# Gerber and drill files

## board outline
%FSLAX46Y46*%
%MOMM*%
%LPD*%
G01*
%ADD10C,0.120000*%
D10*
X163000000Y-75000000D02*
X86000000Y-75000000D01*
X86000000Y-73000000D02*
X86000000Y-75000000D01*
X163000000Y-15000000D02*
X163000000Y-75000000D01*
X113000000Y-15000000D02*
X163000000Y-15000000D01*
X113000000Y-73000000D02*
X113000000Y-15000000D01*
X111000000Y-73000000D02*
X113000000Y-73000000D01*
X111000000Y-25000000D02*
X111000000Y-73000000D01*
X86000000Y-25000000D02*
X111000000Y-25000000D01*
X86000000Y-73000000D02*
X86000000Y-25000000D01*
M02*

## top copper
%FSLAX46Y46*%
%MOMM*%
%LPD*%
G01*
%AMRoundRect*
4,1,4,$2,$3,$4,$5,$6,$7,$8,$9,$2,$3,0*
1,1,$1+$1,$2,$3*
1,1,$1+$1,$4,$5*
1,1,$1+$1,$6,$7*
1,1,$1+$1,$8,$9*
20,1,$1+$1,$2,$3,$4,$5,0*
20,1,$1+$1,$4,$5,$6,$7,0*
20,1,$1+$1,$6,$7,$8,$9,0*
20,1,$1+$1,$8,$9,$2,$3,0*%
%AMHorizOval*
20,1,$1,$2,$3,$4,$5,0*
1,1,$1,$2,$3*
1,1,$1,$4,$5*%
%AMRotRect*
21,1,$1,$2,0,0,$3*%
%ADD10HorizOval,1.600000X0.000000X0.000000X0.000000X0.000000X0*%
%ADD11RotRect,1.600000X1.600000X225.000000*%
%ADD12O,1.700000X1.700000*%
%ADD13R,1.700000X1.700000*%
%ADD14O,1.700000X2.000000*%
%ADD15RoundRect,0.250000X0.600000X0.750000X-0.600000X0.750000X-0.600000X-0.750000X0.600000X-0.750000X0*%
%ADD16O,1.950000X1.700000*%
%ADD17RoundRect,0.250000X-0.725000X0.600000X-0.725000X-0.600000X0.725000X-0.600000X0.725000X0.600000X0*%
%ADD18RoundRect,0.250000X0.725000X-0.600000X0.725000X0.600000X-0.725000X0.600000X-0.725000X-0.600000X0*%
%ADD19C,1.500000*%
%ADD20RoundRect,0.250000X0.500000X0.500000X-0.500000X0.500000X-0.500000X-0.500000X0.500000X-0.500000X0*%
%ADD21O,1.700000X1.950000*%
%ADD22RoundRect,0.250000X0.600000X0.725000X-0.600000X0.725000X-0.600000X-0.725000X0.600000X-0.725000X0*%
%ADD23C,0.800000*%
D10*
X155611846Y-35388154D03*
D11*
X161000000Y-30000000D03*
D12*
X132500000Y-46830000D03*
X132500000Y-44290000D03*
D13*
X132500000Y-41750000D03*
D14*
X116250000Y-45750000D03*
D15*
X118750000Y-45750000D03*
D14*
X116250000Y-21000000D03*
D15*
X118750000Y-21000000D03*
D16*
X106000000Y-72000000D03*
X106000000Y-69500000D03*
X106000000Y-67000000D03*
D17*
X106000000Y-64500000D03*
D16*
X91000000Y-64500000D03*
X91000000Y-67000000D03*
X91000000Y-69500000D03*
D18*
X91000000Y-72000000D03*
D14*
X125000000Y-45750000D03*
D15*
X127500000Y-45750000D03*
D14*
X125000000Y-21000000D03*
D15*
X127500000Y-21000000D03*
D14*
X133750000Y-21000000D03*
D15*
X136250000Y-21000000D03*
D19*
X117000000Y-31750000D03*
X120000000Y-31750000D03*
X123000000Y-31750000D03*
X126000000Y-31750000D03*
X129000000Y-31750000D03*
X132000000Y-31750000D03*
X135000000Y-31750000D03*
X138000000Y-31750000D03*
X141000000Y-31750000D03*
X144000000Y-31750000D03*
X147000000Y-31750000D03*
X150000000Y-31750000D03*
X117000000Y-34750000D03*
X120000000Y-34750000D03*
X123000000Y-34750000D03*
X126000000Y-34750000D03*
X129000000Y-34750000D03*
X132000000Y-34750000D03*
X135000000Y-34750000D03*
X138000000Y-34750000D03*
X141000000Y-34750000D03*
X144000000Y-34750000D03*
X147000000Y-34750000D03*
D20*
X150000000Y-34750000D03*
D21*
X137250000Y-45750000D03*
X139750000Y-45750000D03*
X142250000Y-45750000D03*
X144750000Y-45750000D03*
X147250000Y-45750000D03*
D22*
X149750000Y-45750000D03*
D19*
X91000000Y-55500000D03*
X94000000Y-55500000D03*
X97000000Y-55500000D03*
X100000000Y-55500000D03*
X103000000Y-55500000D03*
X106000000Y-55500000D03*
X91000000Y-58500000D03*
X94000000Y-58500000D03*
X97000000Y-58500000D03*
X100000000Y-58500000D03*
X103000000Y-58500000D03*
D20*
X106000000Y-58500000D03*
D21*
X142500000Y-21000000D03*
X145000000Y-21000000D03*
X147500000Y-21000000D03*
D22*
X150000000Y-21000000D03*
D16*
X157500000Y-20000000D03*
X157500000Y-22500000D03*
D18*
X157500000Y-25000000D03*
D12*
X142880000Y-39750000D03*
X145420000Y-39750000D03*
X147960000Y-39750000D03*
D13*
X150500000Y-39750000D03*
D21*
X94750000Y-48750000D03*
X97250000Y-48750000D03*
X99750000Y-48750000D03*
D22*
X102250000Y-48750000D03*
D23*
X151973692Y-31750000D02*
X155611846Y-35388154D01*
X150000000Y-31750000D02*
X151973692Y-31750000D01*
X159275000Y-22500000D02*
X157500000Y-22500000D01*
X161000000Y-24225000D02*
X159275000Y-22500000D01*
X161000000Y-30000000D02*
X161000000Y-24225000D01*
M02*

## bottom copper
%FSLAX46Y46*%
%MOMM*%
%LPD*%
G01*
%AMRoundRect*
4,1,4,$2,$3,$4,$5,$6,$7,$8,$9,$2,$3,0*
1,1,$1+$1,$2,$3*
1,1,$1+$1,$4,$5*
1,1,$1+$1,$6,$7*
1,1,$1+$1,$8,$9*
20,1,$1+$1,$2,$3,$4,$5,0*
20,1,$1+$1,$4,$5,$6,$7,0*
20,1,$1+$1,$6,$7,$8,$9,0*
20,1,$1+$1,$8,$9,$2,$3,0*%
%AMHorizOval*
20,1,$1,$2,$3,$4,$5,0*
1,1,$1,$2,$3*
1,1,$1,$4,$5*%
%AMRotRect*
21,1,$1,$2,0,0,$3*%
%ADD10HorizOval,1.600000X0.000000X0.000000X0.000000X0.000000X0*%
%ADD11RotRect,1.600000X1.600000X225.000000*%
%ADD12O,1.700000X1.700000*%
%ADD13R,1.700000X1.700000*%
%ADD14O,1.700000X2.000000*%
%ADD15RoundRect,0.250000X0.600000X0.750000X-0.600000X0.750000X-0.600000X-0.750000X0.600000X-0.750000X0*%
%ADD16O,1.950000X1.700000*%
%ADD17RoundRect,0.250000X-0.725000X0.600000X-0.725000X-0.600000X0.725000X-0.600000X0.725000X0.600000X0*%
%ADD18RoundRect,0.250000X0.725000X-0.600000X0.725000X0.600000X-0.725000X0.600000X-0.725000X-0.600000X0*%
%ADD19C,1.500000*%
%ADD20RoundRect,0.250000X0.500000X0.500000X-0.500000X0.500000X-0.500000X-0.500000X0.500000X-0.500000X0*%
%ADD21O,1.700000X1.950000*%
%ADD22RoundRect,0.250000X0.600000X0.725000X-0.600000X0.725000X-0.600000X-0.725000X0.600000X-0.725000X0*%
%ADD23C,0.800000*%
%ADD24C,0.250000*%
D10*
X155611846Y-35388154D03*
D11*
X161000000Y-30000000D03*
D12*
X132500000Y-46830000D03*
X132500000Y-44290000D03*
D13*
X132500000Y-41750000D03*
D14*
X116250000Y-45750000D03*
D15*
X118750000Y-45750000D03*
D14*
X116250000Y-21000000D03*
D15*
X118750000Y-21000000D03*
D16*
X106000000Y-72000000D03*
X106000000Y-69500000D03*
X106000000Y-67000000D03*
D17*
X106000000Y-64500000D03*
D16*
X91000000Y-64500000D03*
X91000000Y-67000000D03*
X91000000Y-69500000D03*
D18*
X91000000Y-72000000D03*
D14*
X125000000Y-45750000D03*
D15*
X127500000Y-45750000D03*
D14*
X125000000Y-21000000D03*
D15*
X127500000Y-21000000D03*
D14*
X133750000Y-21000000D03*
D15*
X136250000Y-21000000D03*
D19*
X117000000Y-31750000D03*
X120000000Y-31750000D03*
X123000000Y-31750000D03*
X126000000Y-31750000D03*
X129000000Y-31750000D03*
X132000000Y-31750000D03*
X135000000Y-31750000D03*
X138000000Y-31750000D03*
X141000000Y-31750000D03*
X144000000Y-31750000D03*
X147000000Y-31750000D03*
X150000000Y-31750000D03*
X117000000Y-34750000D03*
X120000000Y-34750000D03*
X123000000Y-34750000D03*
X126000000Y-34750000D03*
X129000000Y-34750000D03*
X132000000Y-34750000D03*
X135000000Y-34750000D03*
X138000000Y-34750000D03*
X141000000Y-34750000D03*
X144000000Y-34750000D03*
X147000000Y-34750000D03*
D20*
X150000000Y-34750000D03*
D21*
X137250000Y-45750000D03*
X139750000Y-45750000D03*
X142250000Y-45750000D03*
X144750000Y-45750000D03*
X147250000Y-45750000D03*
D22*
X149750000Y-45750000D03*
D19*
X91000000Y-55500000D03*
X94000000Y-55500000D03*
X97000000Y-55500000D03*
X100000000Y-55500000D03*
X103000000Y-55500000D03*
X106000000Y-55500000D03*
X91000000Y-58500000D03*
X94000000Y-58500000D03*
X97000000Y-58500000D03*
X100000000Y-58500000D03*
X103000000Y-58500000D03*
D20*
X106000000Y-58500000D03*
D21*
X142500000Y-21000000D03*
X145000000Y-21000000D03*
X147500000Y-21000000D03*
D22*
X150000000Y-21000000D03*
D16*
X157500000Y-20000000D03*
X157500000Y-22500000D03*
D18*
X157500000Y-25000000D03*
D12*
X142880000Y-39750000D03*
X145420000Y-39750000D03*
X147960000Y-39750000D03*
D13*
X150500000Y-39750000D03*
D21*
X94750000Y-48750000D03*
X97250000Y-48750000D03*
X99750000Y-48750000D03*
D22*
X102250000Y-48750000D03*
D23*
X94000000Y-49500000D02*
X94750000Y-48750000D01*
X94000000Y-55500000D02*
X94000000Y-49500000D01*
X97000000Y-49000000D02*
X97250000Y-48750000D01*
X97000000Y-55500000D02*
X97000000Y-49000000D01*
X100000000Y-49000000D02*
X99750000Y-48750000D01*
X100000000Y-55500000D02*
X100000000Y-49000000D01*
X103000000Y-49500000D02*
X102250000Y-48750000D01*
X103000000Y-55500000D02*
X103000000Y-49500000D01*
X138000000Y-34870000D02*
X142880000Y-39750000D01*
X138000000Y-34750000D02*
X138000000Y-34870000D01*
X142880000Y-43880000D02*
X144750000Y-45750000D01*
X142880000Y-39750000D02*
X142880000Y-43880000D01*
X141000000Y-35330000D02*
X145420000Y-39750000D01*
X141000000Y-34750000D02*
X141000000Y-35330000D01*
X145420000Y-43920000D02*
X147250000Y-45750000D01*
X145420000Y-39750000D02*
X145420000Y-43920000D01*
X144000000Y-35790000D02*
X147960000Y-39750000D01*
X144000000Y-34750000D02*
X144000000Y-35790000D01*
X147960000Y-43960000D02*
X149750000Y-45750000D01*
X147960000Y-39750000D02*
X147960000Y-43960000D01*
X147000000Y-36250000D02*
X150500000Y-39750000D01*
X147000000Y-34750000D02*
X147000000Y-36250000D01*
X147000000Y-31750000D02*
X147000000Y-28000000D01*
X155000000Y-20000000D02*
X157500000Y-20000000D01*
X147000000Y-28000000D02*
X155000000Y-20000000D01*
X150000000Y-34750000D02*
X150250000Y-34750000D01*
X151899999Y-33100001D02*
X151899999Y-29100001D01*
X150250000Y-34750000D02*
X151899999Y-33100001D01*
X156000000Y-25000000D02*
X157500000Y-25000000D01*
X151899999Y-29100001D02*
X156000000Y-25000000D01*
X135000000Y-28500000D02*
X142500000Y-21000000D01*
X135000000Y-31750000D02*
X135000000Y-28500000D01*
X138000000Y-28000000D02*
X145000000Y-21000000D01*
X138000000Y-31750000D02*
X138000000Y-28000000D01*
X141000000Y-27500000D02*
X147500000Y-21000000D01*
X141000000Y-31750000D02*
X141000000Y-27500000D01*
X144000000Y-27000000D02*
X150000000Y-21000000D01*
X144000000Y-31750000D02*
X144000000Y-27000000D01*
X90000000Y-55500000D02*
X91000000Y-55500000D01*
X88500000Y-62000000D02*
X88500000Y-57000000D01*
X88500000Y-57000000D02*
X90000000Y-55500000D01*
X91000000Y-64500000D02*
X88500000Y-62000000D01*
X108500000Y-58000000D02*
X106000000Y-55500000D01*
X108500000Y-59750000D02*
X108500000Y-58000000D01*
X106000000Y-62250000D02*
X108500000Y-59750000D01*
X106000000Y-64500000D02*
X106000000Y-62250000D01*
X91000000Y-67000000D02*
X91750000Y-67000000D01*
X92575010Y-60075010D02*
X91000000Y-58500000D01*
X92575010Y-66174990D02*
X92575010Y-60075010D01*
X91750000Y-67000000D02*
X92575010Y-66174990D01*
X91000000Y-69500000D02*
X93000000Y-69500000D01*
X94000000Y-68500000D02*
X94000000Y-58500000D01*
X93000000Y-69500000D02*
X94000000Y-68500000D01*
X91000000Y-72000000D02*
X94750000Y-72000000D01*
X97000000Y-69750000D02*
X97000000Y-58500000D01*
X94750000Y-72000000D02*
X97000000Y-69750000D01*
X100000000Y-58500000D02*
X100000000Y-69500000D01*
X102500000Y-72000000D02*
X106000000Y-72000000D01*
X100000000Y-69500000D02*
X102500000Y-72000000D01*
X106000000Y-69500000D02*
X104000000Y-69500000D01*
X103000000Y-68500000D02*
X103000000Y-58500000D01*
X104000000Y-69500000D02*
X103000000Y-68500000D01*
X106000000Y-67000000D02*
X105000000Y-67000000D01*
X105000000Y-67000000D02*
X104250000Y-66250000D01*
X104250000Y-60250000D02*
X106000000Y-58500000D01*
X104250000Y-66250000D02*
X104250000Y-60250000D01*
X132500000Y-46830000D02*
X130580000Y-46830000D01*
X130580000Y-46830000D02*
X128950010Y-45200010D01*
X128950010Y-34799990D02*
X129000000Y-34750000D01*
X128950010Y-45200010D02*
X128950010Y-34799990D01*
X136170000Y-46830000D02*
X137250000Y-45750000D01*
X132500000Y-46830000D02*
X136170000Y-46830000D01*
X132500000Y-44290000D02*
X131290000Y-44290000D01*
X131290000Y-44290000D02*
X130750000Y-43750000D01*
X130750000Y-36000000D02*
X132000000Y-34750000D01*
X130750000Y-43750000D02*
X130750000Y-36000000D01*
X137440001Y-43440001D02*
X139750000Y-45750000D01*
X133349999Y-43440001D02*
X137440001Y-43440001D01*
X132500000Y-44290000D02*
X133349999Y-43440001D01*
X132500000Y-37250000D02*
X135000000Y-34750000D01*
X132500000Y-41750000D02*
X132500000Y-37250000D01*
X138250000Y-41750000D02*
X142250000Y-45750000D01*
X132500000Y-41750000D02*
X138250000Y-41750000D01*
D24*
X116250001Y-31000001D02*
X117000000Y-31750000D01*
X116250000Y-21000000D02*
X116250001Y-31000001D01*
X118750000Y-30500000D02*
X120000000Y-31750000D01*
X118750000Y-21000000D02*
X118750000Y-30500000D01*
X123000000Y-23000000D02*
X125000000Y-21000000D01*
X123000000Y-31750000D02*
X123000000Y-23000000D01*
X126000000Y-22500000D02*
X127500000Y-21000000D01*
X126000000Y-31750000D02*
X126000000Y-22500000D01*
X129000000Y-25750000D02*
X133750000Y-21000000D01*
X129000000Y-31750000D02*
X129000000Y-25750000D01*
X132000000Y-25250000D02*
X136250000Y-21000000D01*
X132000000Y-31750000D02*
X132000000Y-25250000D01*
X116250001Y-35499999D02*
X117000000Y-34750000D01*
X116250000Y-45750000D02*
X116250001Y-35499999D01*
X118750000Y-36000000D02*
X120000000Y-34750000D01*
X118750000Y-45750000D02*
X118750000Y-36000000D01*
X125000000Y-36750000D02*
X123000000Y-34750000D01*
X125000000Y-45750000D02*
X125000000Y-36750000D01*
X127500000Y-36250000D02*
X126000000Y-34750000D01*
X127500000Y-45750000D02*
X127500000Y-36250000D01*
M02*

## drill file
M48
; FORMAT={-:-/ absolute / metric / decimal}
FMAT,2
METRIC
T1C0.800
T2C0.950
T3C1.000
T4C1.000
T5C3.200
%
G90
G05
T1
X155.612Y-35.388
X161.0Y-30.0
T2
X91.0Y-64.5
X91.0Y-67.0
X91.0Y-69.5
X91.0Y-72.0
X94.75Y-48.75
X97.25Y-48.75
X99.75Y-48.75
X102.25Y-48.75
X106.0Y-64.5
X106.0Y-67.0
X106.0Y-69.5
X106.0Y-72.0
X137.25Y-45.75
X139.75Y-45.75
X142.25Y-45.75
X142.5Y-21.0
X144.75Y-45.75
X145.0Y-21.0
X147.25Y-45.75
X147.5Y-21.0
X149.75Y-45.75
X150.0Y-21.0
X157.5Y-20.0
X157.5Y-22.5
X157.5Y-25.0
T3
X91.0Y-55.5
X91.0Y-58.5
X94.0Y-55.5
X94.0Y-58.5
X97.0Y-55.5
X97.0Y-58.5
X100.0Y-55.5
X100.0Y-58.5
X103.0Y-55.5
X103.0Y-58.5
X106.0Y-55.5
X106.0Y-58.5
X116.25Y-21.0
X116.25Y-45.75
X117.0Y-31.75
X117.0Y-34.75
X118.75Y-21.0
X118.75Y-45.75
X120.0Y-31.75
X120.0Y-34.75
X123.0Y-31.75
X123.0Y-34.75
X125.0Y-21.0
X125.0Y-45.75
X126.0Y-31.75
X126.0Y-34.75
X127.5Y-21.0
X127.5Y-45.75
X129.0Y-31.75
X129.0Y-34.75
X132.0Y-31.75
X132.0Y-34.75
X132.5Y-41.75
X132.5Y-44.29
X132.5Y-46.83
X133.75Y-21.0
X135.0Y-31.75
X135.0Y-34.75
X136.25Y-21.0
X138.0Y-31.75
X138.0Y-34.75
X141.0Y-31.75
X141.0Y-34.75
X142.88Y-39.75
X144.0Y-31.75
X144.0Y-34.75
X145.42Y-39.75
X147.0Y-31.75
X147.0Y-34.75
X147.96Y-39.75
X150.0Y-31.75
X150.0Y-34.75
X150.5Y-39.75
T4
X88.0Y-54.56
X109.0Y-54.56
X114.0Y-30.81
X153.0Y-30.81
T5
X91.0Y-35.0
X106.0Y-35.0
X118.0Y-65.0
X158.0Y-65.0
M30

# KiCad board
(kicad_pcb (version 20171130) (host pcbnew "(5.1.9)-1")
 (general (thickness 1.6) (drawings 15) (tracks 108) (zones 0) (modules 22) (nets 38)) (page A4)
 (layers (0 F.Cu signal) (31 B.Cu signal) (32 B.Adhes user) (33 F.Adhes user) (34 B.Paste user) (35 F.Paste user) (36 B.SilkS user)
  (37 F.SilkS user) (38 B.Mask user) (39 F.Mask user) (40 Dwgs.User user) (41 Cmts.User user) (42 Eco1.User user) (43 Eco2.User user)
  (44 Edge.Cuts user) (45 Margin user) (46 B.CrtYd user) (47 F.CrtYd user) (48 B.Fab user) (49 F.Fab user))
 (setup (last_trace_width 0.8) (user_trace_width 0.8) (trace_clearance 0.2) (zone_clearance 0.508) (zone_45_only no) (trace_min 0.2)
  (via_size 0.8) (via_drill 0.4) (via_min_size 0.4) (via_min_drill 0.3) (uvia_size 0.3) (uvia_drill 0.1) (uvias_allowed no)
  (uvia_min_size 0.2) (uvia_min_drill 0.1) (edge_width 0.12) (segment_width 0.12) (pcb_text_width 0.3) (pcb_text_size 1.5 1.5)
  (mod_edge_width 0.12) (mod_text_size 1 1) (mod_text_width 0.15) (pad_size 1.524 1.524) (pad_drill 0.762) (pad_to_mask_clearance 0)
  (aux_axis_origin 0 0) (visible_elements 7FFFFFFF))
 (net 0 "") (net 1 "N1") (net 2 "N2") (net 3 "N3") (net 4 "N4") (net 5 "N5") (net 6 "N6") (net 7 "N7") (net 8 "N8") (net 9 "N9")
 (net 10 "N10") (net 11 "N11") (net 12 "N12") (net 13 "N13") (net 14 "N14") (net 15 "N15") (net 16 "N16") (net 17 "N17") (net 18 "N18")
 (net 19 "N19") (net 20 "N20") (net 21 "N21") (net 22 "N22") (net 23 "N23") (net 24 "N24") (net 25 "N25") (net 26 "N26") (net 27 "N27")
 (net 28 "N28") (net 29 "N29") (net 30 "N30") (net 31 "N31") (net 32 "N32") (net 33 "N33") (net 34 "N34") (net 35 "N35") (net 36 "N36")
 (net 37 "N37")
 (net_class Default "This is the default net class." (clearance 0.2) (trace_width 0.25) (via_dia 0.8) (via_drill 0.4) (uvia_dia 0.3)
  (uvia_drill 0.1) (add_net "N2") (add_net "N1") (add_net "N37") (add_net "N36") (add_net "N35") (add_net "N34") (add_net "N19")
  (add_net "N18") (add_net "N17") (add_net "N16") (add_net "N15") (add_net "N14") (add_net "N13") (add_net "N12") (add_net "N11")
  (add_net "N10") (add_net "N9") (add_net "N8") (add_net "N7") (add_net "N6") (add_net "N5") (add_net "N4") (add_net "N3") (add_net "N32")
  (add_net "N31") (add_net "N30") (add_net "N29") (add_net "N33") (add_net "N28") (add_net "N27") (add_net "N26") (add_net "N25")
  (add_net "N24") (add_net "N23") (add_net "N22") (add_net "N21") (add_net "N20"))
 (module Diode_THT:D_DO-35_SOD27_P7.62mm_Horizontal (layer F.Cu) (at 161 30 225)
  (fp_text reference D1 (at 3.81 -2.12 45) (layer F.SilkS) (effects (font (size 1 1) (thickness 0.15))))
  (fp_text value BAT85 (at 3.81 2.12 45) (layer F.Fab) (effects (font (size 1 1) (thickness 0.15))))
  (pad 2 thru_hole oval (at 7.62 0 225) (size 1.6 1.6) (drill 0.8) (layers *.Cu *.Mask) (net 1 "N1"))
  (pad 1 thru_hole rect (at 0 0 225) (size 1.6 1.6) (drill 0.8) (layers *.Cu *.Mask) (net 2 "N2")))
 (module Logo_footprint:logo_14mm (layer F.Cu) (at 98.5 37)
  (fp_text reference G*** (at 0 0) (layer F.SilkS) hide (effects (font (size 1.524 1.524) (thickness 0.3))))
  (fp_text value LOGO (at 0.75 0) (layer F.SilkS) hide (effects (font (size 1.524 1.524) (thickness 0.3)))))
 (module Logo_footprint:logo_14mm (layer F.Cu) (at 137.25 65.25)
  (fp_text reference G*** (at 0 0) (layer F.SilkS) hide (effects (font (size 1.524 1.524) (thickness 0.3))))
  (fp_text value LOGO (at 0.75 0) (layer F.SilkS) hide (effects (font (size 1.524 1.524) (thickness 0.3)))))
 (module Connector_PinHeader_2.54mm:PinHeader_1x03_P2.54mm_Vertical (layer F.Cu) (at 132.5 41.75)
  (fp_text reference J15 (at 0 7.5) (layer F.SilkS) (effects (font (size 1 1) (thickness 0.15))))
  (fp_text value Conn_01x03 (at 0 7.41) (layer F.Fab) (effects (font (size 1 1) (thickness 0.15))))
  (pad 3 thru_hole oval (at 0 5.08) (size 1.7 1.7) (drill 1) (layers *.Cu *.Mask) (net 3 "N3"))
  (pad 2 thru_hole oval (at 0 2.54) (size 1.7 1.7) (drill 1) (layers *.Cu *.Mask) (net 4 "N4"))
  (pad 1 thru_hole rect (at 0 0) (size 1.7 1.7) (drill 1) (layers *.Cu *.Mask) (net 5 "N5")))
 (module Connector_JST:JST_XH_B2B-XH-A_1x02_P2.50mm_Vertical (layer F.Cu) (at 118.75 45.75 180)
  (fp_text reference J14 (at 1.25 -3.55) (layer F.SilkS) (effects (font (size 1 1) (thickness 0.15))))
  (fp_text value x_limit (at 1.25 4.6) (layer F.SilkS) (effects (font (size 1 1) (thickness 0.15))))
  (pad 2 thru_hole oval (at 2.5 0 180) (size 1.7 2) (drill 1) (layers *.Cu *.Mask) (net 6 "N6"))
  (pad 1 thru_hole roundrect (at 0 0 180) (size 1.7 2) (drill 1) (layers *.Cu *.Mask) (roundrect_rratio 0.1470588235294118) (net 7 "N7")))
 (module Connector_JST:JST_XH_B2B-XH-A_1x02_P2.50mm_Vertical (layer F.Cu) (at 118.75 21 180)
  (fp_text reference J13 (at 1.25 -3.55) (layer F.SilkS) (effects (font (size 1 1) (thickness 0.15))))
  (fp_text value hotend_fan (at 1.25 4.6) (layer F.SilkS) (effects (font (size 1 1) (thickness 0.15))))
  (pad 2 thru_hole oval (at 2.5 0 180) (size 1.7 2) (drill 1) (layers *.Cu *.Mask) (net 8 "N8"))
  (pad 1 thru_hole roundrect (at 0 0 180) (size 1.7 2) (drill 1) (layers *.Cu *.Mask) (roundrect_rratio 0.1470588235294118) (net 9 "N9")))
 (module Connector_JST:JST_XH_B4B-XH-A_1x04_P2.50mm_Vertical (layer F.Cu) (at 106 64.5 270)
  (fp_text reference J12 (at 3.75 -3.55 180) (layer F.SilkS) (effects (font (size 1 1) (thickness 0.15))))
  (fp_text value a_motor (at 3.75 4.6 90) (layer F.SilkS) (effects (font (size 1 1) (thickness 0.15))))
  (pad 4 thru_hole oval (at 7.5 0 270) (size 1.7 1.95) (drill 0.95) (layers *.Cu *.Mask) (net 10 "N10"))
  (pad 3 thru_hole oval (at 5 0 270) (size 1.7 1.95) (drill 0.95) (layers *.Cu *.Mask) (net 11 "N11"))
  (pad 2 thru_hole oval (at 2.5 0 270) (size 1.7 1.95) (drill 0.95) (layers *.Cu *.Mask) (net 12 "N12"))
  (pad 1 thru_hole roundrect (at 0 0 270) (size 1.7 1.95) (drill 0.95) (layers *.Cu *.Mask) (roundrect_rratio 0.1470588235294118)
   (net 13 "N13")))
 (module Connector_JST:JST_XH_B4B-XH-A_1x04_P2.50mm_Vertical (layer F.Cu) (at 91 72 90)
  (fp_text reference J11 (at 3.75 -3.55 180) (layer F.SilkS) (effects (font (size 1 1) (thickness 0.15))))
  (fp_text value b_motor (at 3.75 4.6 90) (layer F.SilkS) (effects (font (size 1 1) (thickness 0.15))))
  (pad 4 thru_hole oval (at 7.5 0 90) (size 1.7 1.95) (drill 0.95) (layers *.Cu *.Mask) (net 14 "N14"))
  (pad 3 thru_hole oval (at 5 0 90) (size 1.7 1.95) (drill 0.95) (layers *.Cu *.Mask) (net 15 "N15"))
  (pad 2 thru_hole oval (at 2.5 0 90) (size 1.7 1.95) (drill 0.95) (layers *.Cu *.Mask) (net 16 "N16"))
  (pad 1 thru_hole roundrect (at 0 0 90) (size 1.7 1.95) (drill 0.95) (layers *.Cu *.Mask) (roundrect_rratio 0.1470588235294118)
   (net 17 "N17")))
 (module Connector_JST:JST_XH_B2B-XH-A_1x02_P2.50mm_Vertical (layer F.Cu) (at 127.5 45.75 180)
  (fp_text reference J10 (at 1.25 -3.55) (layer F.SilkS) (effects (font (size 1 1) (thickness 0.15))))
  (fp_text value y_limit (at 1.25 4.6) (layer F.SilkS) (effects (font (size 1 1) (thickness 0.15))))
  (pad 2 thru_hole oval (at 2.5 0 180) (size 1.7 2) (drill 1) (layers *.Cu *.Mask) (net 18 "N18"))
  (pad 1 thru_hole roundrect (at 0 0 180) (size 1.7 2) (drill 1) (layers *.Cu *.Mask) (roundrect_rratio 0.1470588235294118) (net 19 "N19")))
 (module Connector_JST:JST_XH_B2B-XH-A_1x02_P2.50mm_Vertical (layer F.Cu) (at 127.5 21 180)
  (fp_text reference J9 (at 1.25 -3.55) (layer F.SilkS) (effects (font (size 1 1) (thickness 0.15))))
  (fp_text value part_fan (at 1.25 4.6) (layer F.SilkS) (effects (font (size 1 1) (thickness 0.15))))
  (pad 2 thru_hole oval (at 2.5 0 180) (size 1.7 2) (drill 1) (layers *.Cu *.Mask) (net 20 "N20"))
  (pad 1 thru_hole roundrect (at 0 0 180) (size 1.7 2) (drill 1) (layers *.Cu *.Mask) (roundrect_rratio 0.1470588235294118) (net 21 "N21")))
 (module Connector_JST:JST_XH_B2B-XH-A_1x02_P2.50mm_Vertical (layer F.Cu) (at 136.25 21 180)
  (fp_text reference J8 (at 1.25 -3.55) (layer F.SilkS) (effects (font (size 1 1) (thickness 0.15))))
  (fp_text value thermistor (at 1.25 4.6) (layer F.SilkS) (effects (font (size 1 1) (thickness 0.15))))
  (pad 2 thru_hole oval (at 2.5 0 180) (size 1.7 2) (drill 1) (layers *.Cu *.Mask) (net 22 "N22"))
  (pad 1 thru_hole roundrect (at 0 0 180) (size 1.7 2) (drill 1) (layers *.Cu *.Mask) (roundrect_rratio 0.1470588235294118) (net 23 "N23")))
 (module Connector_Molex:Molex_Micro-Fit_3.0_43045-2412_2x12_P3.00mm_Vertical (layer F.Cu) (at 150 34.75 180)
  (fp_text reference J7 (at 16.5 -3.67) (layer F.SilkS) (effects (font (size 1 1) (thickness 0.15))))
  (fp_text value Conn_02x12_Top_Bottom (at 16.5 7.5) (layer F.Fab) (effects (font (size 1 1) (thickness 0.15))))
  (pad 24 thru_hole circle (at 33 3 180) (size 1.5 1.5) (drill 1) (layers *.Cu *.Mask) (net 8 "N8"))
  (pad 23 thru_hole circle (at 30 3 180) (size 1.5 1.5) (drill 1) (layers *.Cu *.Mask) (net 9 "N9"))
  (pad 22 thru_hole circle (at 27 3 180) (size 1.5 1.5) (drill 1) (layers *.Cu *.Mask) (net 20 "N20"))
  (pad 21 thru_hole circle (at 24 3 180) (size 1.5 1.5) (drill 1) (layers *.Cu *.Mask) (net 21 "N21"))
  (pad 20 thru_hole circle (at 21 3 180) (size 1.5 1.5) (drill 1) (layers *.Cu *.Mask) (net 22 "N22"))
  (pad 19 thru_hole circle (at 18 3 180) (size 1.5 1.5) (drill 1) (layers *.Cu *.Mask) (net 23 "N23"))
  (pad 18 thru_hole circle (at 15 3 180) (size 1.5 1.5) (drill 1) (layers *.Cu *.Mask) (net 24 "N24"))
  (pad 17 thru_hole circle (at 12 3 180) (size 1.5 1.5) (drill 1) (layers *.Cu *.Mask) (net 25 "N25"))
  (pad 16 thru_hole circle (at 9 3 180) (size 1.5 1.5) (drill 1) (layers *.Cu *.Mask) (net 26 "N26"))
  (pad 15 thru_hole circle (at 6 3 180) (size 1.5 1.5) (drill 1) (layers *.Cu *.Mask) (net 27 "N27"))
  (pad 14 thru_hole circle (at 3 3 180) (size 1.5 1.5) (drill 1) (layers *.Cu *.Mask) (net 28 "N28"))
  (pad 13 thru_hole circle (at 0 3 180) (size 1.5 1.5) (drill 1) (layers *.Cu *.Mask) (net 1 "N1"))
  (pad 12 thru_hole circle (at 33 0 180) (size 1.5 1.5) (drill 1) (layers *.Cu *.Mask) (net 6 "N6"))
  (pad 11 thru_hole circle (at 30 0 180) (size 1.5 1.5) (drill 1) (layers *.Cu *.Mask) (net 7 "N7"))
  (pad 10 thru_hole circle (at 27 0 180) (size 1.5 1.5) (drill 1) (layers *.Cu *.Mask) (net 18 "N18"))
  (pad 9 thru_hole circle (at 24 0 180) (size 1.5 1.5) (drill 1) (layers *.Cu *.Mask) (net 19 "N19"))
  (pad 8 thru_hole circle (at 21 0 180) (size 1.5 1.5) (drill 1) (layers *.Cu *.Mask) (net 3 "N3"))
  (pad 7 thru_hole circle (at 18 0 180) (size 1.5 1.5) (drill 1) (layers *.Cu *.Mask) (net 4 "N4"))
  (pad 6 thru_hole circle (at 15 0 180) (size 1.5 1.5) (drill 1) (layers *.Cu *.Mask) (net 5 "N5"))
  (pad 5 thru_hole circle (at 12 0 180) (size 1.5 1.5) (drill 1) (layers *.Cu *.Mask) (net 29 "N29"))
  (pad 4 thru_hole circle (at 9 0 180) (size 1.5 1.5) (drill 1) (layers *.Cu *.Mask) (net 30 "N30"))
  (pad 3 thru_hole circle (at 6 0 180) (size 1.5 1.5) (drill 1) (layers *.Cu *.Mask) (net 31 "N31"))
  (pad 2 thru_hole circle (at 3 0 180) (size 1.5 1.5) (drill 1) (layers *.Cu *.Mask) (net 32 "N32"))
  (pad 1 thru_hole roundrect (at 0 0 180) (size 1.5 1.5) (drill 1) (layers *.Cu *.Mask) (roundrect_rratio 0.1666666666666667) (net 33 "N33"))
  (pad "" np_thru_hole circle (at 36 3.94 180) (size 1 1) (drill 1) (layers *.Cu *.Mask))
  (pad "" np_thru_hole circle (at -3 3.94 180) (size 1 1) (drill 1) (layers *.Cu *.Mask)))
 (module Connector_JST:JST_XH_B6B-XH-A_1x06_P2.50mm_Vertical (layer F.Cu) (at 149.75 45.75 180)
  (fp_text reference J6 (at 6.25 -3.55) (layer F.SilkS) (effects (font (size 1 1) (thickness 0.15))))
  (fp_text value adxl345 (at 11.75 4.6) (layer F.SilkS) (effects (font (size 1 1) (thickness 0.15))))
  (pad 6 thru_hole oval (at 12.5 0 180) (size 1.7 1.95) (drill 0.95) (layers *.Cu *.Mask) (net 3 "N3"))
  (pad 5 thru_hole oval (at 10 0 180) (size 1.7 1.95) (drill 0.95) (layers *.Cu *.Mask) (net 4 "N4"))
  (pad 4 thru_hole oval (at 7.5 0 180) (size 1.7 1.95) (drill 0.95) (layers *.Cu *.Mask) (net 5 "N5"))
  (pad 3 thru_hole oval (at 5 0 180) (size 1.7 1.95) (drill 0.95) (layers *.Cu *.Mask) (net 29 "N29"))
  (pad 2 thru_hole oval (at 2.5 0 180) (size 1.7 1.95) (drill 0.95) (layers *.Cu *.Mask) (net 30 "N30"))
  (pad 1 thru_hole roundrect (at 0 0 180) (size 1.7 1.95) (drill 0.95) (layers *.Cu *.Mask) (roundrect_rratio 0.1470588235294118)
   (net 31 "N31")))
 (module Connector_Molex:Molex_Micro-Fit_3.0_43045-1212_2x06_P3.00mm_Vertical (layer F.Cu) (at 106 58.5 180)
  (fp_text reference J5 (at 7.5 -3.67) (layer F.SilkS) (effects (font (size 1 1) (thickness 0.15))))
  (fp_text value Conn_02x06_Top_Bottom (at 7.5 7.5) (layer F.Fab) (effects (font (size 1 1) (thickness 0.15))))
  (pad 12 thru_hole circle (at 15 3 180) (size 1.5 1.5) (drill 1) (layers *.Cu *.Mask) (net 14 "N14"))
  (pad 11 thru_hole circle (at 12 3 180) (size 1.5 1.5) (drill 1) (layers *.Cu *.Mask) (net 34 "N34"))
  (pad 10 thru_hole circle (at 9 3 180) (size 1.5 1.5) (drill 1) (layers *.Cu *.Mask) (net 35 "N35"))
  (pad 9 thru_hole circle (at 6 3 180) (size 1.5 1.5) (drill 1) (layers *.Cu *.Mask) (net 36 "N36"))
  (pad 8 thru_hole circle (at 3 3 180) (size 1.5 1.5) (drill 1) (layers *.Cu *.Mask) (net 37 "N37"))
  (pad 7 thru_hole circle (at 0 3 180) (size 1.5 1.5) (drill 1) (layers *.Cu *.Mask) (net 13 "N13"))
  (pad 6 thru_hole circle (at 15 0 180) (size 1.5 1.5) (drill 1) (layers *.Cu *.Mask) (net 15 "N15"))
  (pad 5 thru_hole circle (at 12 0 180) (size 1.5 1.5) (drill 1) (layers *.Cu *.Mask) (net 16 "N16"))
  (pad 4 thru_hole circle (at 9 0 180) (size 1.5 1.5) (drill 1) (layers *.Cu *.Mask) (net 17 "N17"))
  (pad 3 thru_hole circle (at 6 0 180) (size 1.5 1.5) (drill 1) (layers *.Cu *.Mask) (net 10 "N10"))
  (pad 2 thru_hole circle (at 3 0 180) (size 1.5 1.5) (drill 1) (layers *.Cu *.Mask) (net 11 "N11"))
  (pad 1 thru_hole roundrect (at 0 0 180) (size 1.5 1.5) (drill 1) (layers *.Cu *.Mask) (roundrect_rratio 0.1666666666666667) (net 12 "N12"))
  (pad "" np_thru_hole circle (at 18 3.94 180) (size 1 1) (drill 1) (layers *.Cu *.Mask))
  (pad "" np_thru_hole circle (at -3 3.94 180) (size 1 1) (drill 1) (layers *.Cu *.Mask)))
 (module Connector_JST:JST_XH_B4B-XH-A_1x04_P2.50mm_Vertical (layer F.Cu) (at 150 21 180)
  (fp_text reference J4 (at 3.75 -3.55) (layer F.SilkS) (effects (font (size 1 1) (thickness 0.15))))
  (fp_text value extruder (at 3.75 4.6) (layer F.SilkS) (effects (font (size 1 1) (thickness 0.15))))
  (pad 4 thru_hole oval (at 7.5 0 180) (size 1.7 1.95) (drill 0.95) (layers *.Cu *.Mask) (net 24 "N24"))
  (pad 3 thru_hole oval (at 5 0 180) (size 1.7 1.95) (drill 0.95) (layers *.Cu *.Mask) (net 25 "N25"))
  (pad 2 thru_hole oval (at 2.5 0 180) (size 1.7 1.95) (drill 0.95) (layers *.Cu *.Mask) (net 26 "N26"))
  (pad 1 thru_hole roundrect (at 0 0 180) (size 1.7 1.95) (drill 0.95) (layers *.Cu *.Mask) (roundrect_rratio 0.1470588235294118)
   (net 27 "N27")))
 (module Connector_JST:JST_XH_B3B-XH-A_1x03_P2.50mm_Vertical (layer F.Cu) (at 157.5 25 90)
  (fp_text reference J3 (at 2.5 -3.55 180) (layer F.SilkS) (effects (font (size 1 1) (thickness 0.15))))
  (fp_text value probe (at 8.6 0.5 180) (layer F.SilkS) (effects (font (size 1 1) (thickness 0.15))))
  (pad 3 thru_hole oval (at 5 0 90) (size 1.7 1.95) (drill 0.95) (layers *.Cu *.Mask) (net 28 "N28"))
  (pad 2 thru_hole oval (at 2.5 0 90) (size 1.7 1.95) (drill 0.95) (layers *.Cu *.Mask) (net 2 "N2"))
  (pad 1 thru_hole roundrect (at 0 0 90) (size 1.7 1.95) (drill 0.95) (layers *.Cu *.Mask) (roundrect_rratio 0.1470588235294118)
   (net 33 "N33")))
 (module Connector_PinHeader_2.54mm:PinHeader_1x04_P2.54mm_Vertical (layer F.Cu) (at 150.5 39.75 270)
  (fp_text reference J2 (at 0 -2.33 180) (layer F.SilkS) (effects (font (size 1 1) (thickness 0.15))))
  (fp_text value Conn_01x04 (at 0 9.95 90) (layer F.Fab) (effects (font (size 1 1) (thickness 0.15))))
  (pad 4 thru_hole oval (at 0 7.62 270) (size 1.7 1.7) (drill 1) (layers *.Cu *.Mask) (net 29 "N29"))
  (pad 3 thru_hole oval (at 0 5.08 270) (size 1.7 1.7) (drill 1) (layers *.Cu *.Mask) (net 30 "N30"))
  (pad 2 thru_hole oval (at 0 2.54 270) (size 1.7 1.7) (drill 1) (layers *.Cu *.Mask) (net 31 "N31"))
  (pad 1 thru_hole rect (at 0 0 270) (size 1.7 1.7) (drill 1) (layers *.Cu *.Mask) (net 32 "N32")))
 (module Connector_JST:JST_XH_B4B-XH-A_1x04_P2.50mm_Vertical (layer F.Cu) (at 102.25 48.75 180)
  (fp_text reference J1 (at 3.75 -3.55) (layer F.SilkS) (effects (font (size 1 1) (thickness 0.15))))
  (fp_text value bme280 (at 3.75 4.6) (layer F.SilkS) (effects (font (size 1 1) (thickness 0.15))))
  (pad 4 thru_hole oval (at 7.5 0 180) (size 1.7 1.95) (drill 0.95) (layers *.Cu *.Mask) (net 34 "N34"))
  (pad 3 thru_hole oval (at 5 0 180) (size 1.7 1.95) (drill 0.95) (layers *.Cu *.Mask) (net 35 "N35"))
  (pad 2 thru_hole oval (at 2.5 0 180) (size 1.7 1.95) (drill 0.95) (layers *.Cu *.Mask) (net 36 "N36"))
  (pad 1 thru_hole roundrect (at 0 0 180) (size 1.7 1.95) (drill 0.95) (layers *.Cu *.Mask) (roundrect_rratio 0.1470588235294118)
   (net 37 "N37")))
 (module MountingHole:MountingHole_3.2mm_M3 (layer F.Cu) (at 158 65 180)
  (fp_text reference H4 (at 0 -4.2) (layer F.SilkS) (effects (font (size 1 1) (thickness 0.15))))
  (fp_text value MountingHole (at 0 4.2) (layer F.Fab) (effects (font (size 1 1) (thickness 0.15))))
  (pad 1 np_thru_hole circle (at 0 0 180) (size 3.2 3.2) (drill 3.2) (layers *.Cu *.Mask)))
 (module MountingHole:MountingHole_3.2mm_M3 (layer F.Cu) (at 118 65 180)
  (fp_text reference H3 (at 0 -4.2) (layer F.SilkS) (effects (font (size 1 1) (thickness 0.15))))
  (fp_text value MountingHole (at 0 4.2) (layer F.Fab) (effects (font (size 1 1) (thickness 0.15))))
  (pad 1 np_thru_hole circle (at 0 0 180) (size 3.2 3.2) (drill 3.2) (layers *.Cu *.Mask)))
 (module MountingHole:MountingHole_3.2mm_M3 (layer F.Cu) (at 106 35 180)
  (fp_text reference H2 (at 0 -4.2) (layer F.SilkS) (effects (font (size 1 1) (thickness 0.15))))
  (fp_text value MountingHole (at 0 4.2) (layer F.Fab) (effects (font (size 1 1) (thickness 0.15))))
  (pad 1 np_thru_hole circle (at 0 0 180) (size 3.2 3.2) (drill 3.2) (layers *.Cu *.Mask)))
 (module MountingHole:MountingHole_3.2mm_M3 (layer F.Cu) (at 91 35 180)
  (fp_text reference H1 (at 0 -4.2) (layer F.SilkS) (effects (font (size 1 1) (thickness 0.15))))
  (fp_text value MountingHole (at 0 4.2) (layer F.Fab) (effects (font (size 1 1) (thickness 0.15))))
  (pad 1 np_thru_hole circle (at 0 0 180) (size 3.2 3.2) (drill 3.2) (layers *.Cu *.Mask)))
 (gr_line (start 163 75) (end 86 75) (layer Edge.Cuts) (width 0.12))
 (gr_line (start 86 73) (end 86 75) (layer Edge.Cuts) (width 0.12))
 (gr_line (start 163 15) (end 163 75) (layer Edge.Cuts) (width 0.12))
 (gr_line (start 113 15) (end 163 15) (layer Edge.Cuts) (width 0.12))
 (gr_line (start 113 73) (end 113 15) (layer Edge.Cuts) (width 0.12))
 (gr_line (start 111 73) (end 113 73) (layer Edge.Cuts) (width 0.12))
 (gr_line (start 111 25) (end 111 73) (layer Edge.Cuts) (width 0.12))
 (gr_line (start 86 25) (end 111 25) (layer Edge.Cuts) (width 0.12))
 (gr_line (start 86 73) (end 86 25) (layer Edge.Cuts) (width 0.12))
 (segment (start 94 49.5) (end 94.75 48.75) (width 0.8) (layer B.Cu) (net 34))
 (segment (start 94 55.5) (end 94 49.5) (width 0.8) (layer B.Cu) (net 34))
 (segment (start 97 49) (end 97.25 48.75) (width 0.8) (layer B.Cu) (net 35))
 (segment (start 97 55.5) (end 97 49) (width 0.8) (layer B.Cu) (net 35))
 (segment (start 100 49) (end 99.75 48.75) (width 0.8) (layer B.Cu) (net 36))
 (segment (start 100 55.5) (end 100 49) (width 0.8) (layer B.Cu) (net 36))
 (segment (start 103 49.5) (end 102.25 48.75) (width 0.8) (layer B.Cu) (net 37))
 (segment (start 103 55.5) (end 103 49.5) (width 0.8) (layer B.Cu) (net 37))
 (segment (start 138 34.87) (end 142.88 39.75) (width 0.8) (layer B.Cu) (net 29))
 (segment (start 138 34.75) (end 138 34.87) (width 0.8) (layer B.Cu) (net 29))
 (segment (start 142.88 43.88) (end 144.75 45.75) (width 0.8) (layer B.Cu) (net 29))
 (segment (start 142.88 39.75) (end 142.88 43.88) (width 0.8) (layer B.Cu) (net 29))
 (segment (start 141 35.33) (end 145.42 39.75) (width 0.8) (layer B.Cu) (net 30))
 (segment (start 141 34.75) (end 141 35.33) (width 0.8) (layer B.Cu) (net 30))
 (segment (start 145.42 43.92) (end 147.25 45.75) (width 0.8) (layer B.Cu) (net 30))
 (segment (start 145.42 39.75) (end 145.42 43.92) (width 0.8) (layer B.Cu) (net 30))
 (segment (start 144 35.79) (end 147.96 39.75) (width 0.8) (layer B.Cu) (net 31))
 (segment (start 144 34.75) (end 144 35.79) (width 0.8) (layer B.Cu) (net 31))
 (segment (start 147.96 43.96) (end 149.75 45.75) (width 0.8) (layer B.Cu) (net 31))
 (segment (start 147.96 39.75) (end 147.96 43.96) (width 0.8) (layer B.Cu) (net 31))
 (segment (start 147 36.25) (end 150.5 39.75) (width 0.8) (layer B.Cu) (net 32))
 (segment (start 147 34.75) (end 147 36.25) (width 0.8) (layer B.Cu) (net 32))
 (segment (start 147 31.75) (end 147 28) (width 0.8) (layer B.Cu) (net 28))
 (segment (start 155 20) (end 157.5 20) (width 0.8) (layer B.Cu) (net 28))
 (segment (start 147 28) (end 155 20) (width 0.8) (layer B.Cu) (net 28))
 (segment (start 150 34.75) (end 150.25 34.75) (width 0.8) (layer B.Cu) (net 33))
 (segment (start 151.899999 33.100001) (end 151.899999 29.100001) (width 0.8) (layer B.Cu) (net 33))
 (segment (start 150.25 34.75) (end 151.899999 33.100001) (width 0.8) (layer B.Cu) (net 33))
 (segment (start 156 25) (end 157.5 25) (width 0.8) (layer B.Cu) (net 33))
 (segment (start 151.899999 29.100001) (end 156 25) (width 0.8) (layer B.Cu) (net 33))
 (segment (start 135 28.5) (end 142.5 21) (width 0.8) (layer B.Cu) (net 24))
 (segment (start 135 31.75) (end 135 28.5) (width 0.8) (layer B.Cu) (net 24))
 (segment (start 138 28) (end 145 21) (width 0.8) (layer B.Cu) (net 25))
 (segment (start 138 31.75) (end 138 28) (width 0.8) (layer B.Cu) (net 25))
 (segment (start 141 27.5) (end 147.5 21) (width 0.8) (layer B.Cu) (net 26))
 (segment (start 141 31.75) (end 141 27.5) (width 0.8) (layer B.Cu) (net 26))
 (segment (start 144 27) (end 150 21) (width 0.8) (layer B.Cu) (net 27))
 (segment (start 144 31.75) (end 144 27) (width 0.8) (layer B.Cu) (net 27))
 (segment (start 90 55.5) (end 91 55.5) (width 0.8) (layer B.Cu) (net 14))
 (segment (start 88.5 62) (end 88.5 57) (width 0.8) (layer B.Cu) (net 14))
 (segment (start 88.5 57) (end 90 55.5) (width 0.8) (layer B.Cu) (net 14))
 (segment (start 91 64.5) (end 88.5 62) (width 0.8) (layer B.Cu) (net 14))
 (segment (start 108.5 58) (end 106 55.5) (width 0.8) (layer B.Cu) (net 13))
 (segment (start 108.5 59.75) (end 108.5 58) (width 0.8) (layer B.Cu) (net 13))
 (segment (start 106 62.25) (end 108.5 59.75) (width 0.8) (layer B.Cu) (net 13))
 (segment (start 106 64.5) (end 106 62.25) (width 0.8) (layer B.Cu) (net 13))
 (segment (start 91 67) (end 91.75 67) (width 0.8) (layer B.Cu) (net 15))
 (segment (start 92.57501 60.07501) (end 91 58.5) (width 0.8) (layer B.Cu) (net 15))
 (segment (start 92.57501 66.17499) (end 92.57501 60.07501) (width 0.8) (layer B.Cu) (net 15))
 (segment (start 91.75 67) (end 92.57501 66.17499) (width 0.8) (layer B.Cu) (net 15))
 (segment (start 91 69.5) (end 93 69.5) (width 0.8) (layer B.Cu) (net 16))
 (segment (start 94 68.5) (end 94 58.5) (width 0.8) (layer B.Cu) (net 16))
 (segment (start 93 69.5) (end 94 68.5) (width 0.8) (layer B.Cu) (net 16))
 (segment (start 91 72) (end 94.75 72) (width 0.8) (layer B.Cu) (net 17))
 (segment (start 97 69.75) (end 97 58.5) (width 0.8) (layer B.Cu) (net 17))
 (segment (start 94.75 72) (end 97 69.75) (width 0.8) (layer B.Cu) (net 17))
 (segment (start 100 58.5) (end 100 69.5) (width 0.8) (layer B.Cu) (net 10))
 (segment (start 102.5 72) (end 106 72) (width 0.8) (layer B.Cu) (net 10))
 (segment (start 100 69.5) (end 102.5 72) (width 0.8) (layer B.Cu) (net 10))
 (segment (start 106 69.5) (end 104 69.5) (width 0.8) (layer B.Cu) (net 11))
 (segment (start 103 68.5) (end 103 58.5) (width 0.8) (layer B.Cu) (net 11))
 (segment (start 104 69.5) (end 103 68.5) (width 0.8) (layer B.Cu) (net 11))
 (segment (start 106 67) (end 105 67) (width 0.8) (layer B.Cu) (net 12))
 (segment (start 105 67) (end 104.25 66.25) (width 0.8) (layer B.Cu) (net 12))
 (segment (start 104.25 60.25) (end 106 58.5) (width 0.8) (layer B.Cu) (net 12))
 (segment (start 104.25 66.25) (end 104.25 60.25) (width 0.8) (layer B.Cu) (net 12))
 (segment (start 132.5 46.83) (end 130.58 46.83) (width 0.8) (layer B.Cu) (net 3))
 (segment (start 130.58 46.83) (end 128.95001 45.20001) (width 0.8) (layer B.Cu) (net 3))
 (segment (start 128.95001 34.79999) (end 129 34.75) (width 0.8) (layer B.Cu) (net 3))
 (segment (start 128.95001 45.20001) (end 128.95001 34.79999) (width 0.8) (layer B.Cu) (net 3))
 (segment (start 136.17 46.83) (end 137.25 45.75) (width 0.8) (layer B.Cu) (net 3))
 (segment (start 132.5 46.83) (end 136.17 46.83) (width 0.8) (layer B.Cu) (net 3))
 (segment (start 132.5 44.29) (end 131.29 44.29) (width 0.8) (layer B.Cu) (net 4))
 (segment (start 131.29 44.29) (end 130.75 43.75) (width 0.8) (layer B.Cu) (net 4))
 (segment (start 130.75 36) (end 132 34.75) (width 0.8) (layer B.Cu) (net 4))
 (segment (start 130.75 43.75) (end 130.75 36) (width 0.8) (layer B.Cu) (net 4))
 (segment (start 137.440001 43.440001) (end 139.75 45.75) (width 0.8) (layer B.Cu) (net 4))
 (segment (start 133.349999 43.440001) (end 137.440001 43.440001) (width 0.8) (layer B.Cu) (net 4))
 (segment (start 132.5 44.29) (end 133.349999 43.440001) (width 0.8) (layer B.Cu) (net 4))
 (segment (start 132.5 37.25) (end 135 34.75) (width 0.8) (layer B.Cu) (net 5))
 (segment (start 132.5 41.75) (end 132.5 37.25) (width 0.8) (layer B.Cu) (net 5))
 (segment (start 138.25 41.75) (end 142.25 45.75) (width 0.8) (layer B.Cu) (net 5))
 (segment (start 132.5 41.75) (end 138.25 41.75) (width 0.8) (layer B.Cu) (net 5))
 (segment (start 116.250001 31.000001) (end 117 31.75) (width 0.25) (layer B.Cu) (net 8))
 (segment (start 116.25 21) (end 116.250001 31.000001) (width 0.25) (layer B.Cu) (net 8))
 (segment (start 118.75 30.5) (end 120 31.75) (width 0.25) (layer B.Cu) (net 9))
 (segment (start 118.75 21) (end 118.75 30.5) (width 0.25) (layer B.Cu) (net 9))
 (segment (start 123 23) (end 125 21) (width 0.25) (layer B.Cu) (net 20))
 (segment (start 123 31.75) (end 123 23) (width 0.25) (layer B.Cu) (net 20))
 (segment (start 126 22.5) (end 127.5 21) (width 0.25) (layer B.Cu) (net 21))
 (segment (start 126 31.75) (end 126 22.5) (width 0.25) (layer B.Cu) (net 21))
 (segment (start 129 25.75) (end 133.75 21) (width 0.25) (layer B.Cu) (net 22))
 (segment (start 129 31.75) (end 129 25.75) (width 0.25) (layer B.Cu) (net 22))
 (segment (start 132 25.25) (end 136.25 21) (width 0.25) (layer B.Cu) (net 23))
 (segment (start 132 31.75) (end 132 25.25) (width 0.25) (layer B.Cu) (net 23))
 (segment (start 116.250001 35.499999) (end 117 34.75) (width 0.25) (layer B.Cu) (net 6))
 (segment (start 116.25 45.75) (end 116.250001 35.499999) (width 0.25) (layer B.Cu) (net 6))
 (segment (start 118.75 36) (end 120 34.75) (width 0.25) (layer B.Cu) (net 7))
 (segment (start 118.75 45.75) (end 118.75 36) (width 0.25) (layer B.Cu) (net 7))
 (segment (start 125 36.75) (end 123 34.75) (width 0.25) (layer B.Cu) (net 18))
 (segment (start 125 45.75) (end 125 36.75) (width 0.25) (layer B.Cu) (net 18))
 (segment (start 127.5 36.25) (end 126 34.75) (width 0.25) (layer B.Cu) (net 19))
 (segment (start 127.5 45.75) (end 127.5 36.25) (width 0.25) (layer B.Cu) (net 19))
 (segment (start 151.973692 31.75) (end 155.611846 35.388154) (width 0.8) (layer F.Cu) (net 1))
 (segment (start 150 31.75) (end 151.973692 31.75) (width 0.8) (layer F.Cu) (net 1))
 (segment (start 159.275 22.5) (end 157.5 22.5) (width 0.8) (layer F.Cu) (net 2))
 (segment (start 161 24.225) (end 159.275 22.5) (width 0.8) (layer F.Cu) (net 2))
 (segment (start 161 30) (end 161 24.225) (width 0.8) (layer F.Cu) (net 2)))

